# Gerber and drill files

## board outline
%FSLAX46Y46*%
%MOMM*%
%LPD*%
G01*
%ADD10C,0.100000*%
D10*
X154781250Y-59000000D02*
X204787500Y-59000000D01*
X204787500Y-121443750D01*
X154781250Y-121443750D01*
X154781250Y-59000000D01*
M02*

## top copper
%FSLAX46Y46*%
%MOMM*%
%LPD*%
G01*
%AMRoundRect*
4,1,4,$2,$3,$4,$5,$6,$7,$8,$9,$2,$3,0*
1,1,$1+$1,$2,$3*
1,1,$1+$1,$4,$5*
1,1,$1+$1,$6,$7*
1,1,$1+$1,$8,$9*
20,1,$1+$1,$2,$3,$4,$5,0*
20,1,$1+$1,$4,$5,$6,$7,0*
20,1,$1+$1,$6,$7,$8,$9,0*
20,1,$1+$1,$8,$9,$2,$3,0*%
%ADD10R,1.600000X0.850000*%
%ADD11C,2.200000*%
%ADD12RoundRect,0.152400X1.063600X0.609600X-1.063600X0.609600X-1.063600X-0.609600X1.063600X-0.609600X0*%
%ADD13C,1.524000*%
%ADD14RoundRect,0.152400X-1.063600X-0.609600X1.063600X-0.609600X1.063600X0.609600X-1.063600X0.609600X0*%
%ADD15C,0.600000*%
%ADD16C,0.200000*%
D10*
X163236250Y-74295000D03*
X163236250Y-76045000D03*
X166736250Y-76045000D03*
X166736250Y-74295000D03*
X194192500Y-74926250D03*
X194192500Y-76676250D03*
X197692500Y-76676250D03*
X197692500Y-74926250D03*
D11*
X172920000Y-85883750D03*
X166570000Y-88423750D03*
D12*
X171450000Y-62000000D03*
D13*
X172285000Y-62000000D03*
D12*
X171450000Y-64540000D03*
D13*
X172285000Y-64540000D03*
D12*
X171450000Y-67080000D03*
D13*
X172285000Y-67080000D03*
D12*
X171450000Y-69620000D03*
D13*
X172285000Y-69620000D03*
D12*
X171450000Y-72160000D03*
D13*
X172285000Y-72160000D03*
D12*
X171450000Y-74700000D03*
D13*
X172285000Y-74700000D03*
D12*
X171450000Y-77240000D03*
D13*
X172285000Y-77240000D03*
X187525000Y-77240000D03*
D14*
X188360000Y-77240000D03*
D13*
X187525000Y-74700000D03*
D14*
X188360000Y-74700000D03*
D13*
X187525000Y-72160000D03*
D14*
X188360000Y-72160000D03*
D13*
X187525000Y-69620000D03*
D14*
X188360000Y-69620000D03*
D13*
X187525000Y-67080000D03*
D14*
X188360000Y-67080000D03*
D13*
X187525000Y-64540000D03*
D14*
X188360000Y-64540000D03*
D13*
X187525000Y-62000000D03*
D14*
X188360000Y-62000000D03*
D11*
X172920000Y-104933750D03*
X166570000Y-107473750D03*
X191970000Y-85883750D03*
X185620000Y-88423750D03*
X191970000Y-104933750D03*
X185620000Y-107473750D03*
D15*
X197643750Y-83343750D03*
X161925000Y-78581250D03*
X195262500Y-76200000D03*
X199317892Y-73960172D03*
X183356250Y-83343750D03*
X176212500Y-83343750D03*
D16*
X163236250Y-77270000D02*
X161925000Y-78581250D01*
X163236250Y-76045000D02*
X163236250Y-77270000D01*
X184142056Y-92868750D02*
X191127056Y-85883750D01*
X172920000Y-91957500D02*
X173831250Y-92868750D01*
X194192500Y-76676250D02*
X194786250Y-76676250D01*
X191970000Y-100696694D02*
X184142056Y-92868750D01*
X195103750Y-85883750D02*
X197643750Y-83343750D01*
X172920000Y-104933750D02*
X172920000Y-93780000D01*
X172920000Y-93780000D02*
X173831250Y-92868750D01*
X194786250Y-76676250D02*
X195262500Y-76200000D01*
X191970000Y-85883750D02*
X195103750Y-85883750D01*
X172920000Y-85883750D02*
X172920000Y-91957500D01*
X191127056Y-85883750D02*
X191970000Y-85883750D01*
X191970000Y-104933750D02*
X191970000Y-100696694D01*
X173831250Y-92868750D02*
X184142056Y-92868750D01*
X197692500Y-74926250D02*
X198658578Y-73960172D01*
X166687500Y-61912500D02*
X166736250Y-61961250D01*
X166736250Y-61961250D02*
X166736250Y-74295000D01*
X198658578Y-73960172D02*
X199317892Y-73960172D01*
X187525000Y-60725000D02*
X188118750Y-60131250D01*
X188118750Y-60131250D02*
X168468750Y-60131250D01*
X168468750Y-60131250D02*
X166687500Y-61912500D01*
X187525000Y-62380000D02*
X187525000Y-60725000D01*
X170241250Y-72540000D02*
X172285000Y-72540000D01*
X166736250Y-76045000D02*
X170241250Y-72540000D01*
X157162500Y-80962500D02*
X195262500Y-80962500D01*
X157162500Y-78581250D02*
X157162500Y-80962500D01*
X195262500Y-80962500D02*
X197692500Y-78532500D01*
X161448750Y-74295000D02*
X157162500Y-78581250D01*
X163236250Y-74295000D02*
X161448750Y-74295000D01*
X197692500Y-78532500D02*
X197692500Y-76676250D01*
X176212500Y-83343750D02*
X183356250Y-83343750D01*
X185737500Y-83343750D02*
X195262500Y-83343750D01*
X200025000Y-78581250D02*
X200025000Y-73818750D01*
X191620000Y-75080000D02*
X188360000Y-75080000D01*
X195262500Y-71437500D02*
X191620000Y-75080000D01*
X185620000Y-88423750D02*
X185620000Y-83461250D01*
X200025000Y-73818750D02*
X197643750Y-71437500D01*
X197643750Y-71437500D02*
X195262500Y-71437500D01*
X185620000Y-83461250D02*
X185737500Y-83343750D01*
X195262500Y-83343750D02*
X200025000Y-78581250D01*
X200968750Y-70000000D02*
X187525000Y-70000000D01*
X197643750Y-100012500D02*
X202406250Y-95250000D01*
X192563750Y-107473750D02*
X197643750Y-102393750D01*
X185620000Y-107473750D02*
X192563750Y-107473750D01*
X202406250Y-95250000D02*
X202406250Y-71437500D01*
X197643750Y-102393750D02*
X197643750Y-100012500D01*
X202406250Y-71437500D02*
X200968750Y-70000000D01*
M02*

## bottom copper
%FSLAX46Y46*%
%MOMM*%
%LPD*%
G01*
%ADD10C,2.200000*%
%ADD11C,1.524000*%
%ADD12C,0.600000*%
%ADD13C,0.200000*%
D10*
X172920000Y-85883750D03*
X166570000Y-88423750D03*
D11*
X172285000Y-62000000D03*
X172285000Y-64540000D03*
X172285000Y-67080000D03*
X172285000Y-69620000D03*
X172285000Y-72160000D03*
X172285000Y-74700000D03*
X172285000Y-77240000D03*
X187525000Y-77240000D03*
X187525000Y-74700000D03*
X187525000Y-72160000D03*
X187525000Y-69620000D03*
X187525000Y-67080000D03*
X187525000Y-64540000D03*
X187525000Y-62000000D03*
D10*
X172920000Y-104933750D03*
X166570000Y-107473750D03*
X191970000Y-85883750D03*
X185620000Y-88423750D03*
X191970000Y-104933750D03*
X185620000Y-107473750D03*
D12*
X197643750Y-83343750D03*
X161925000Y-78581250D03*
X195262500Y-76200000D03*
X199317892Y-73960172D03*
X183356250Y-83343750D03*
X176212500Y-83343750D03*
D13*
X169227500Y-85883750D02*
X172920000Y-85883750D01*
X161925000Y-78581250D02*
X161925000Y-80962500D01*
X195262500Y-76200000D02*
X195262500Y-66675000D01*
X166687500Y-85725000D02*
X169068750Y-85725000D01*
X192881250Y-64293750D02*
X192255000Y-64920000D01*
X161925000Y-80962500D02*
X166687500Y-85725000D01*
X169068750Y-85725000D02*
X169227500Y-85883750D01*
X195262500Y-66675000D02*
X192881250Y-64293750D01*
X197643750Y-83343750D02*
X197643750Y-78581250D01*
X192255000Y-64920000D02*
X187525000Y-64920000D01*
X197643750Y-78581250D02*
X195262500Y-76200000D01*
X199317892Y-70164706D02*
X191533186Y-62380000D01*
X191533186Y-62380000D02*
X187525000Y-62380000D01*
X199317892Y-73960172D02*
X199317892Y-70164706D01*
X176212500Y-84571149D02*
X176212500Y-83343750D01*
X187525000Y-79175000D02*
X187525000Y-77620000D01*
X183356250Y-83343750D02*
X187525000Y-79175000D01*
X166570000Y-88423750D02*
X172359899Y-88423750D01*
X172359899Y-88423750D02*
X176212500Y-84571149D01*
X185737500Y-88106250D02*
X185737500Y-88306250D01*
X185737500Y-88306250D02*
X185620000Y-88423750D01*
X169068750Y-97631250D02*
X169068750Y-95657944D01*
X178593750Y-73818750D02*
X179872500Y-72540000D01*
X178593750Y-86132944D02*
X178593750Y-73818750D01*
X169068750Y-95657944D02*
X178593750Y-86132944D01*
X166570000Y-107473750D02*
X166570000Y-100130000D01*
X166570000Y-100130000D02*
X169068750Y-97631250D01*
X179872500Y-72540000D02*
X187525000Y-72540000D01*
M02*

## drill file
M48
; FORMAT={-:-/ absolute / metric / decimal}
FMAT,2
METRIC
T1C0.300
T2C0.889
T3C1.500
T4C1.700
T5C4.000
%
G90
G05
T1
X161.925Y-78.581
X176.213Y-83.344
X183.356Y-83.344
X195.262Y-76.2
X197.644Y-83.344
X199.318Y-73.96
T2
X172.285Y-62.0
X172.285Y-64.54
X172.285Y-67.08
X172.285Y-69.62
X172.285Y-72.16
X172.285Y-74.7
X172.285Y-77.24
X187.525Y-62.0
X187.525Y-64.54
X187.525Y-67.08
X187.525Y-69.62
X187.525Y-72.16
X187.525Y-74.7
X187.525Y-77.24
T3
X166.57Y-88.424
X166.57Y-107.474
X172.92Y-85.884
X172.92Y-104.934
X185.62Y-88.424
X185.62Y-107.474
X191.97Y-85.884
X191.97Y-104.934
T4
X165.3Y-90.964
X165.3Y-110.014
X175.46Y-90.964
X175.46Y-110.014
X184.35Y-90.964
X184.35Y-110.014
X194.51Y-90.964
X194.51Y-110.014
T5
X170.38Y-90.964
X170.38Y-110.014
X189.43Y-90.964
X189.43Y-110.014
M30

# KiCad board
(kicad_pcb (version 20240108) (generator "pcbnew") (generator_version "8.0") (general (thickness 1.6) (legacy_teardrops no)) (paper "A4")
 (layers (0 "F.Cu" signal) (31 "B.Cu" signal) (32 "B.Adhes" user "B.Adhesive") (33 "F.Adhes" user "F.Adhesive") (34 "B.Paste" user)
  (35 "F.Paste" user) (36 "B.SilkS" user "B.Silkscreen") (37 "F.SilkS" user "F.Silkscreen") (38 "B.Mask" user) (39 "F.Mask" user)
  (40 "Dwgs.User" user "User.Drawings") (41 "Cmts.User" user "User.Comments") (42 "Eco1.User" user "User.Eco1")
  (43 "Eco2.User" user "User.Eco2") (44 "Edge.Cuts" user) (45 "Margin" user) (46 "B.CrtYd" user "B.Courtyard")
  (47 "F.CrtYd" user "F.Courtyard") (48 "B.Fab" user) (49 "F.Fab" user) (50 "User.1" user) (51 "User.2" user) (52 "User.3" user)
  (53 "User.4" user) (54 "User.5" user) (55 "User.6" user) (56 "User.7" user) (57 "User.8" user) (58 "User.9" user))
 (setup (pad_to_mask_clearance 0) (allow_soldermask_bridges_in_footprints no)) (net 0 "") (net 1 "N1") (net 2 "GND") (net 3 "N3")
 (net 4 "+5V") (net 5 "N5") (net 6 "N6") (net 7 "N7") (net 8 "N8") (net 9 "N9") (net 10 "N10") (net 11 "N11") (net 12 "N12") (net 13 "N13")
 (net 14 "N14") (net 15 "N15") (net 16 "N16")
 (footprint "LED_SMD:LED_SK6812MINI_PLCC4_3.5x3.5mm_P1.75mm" (layer "F.Cu") (at 164.98625 75.17)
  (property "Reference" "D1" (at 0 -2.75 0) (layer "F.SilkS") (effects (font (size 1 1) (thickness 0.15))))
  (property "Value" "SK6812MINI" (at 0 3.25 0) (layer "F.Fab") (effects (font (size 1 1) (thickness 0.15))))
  (pad "1" smd rect (at -1.75 -0.875) (size 1.6 0.85) (layers "F.Cu" "F.Paste" "F.Mask") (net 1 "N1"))
  (pad "2" smd rect (at -1.75 0.875) (size 1.6 0.85) (layers "F.Cu" "F.Paste" "F.Mask") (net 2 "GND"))
  (pad "3" smd rect (at 1.75 0.875) (size 1.6 0.85) (layers "F.Cu" "F.Paste" "F.Mask") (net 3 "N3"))
  (pad "4" smd rect (at 1.75 -0.875) (size 1.6 0.85) (layers "F.Cu" "F.Paste" "F.Mask") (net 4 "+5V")))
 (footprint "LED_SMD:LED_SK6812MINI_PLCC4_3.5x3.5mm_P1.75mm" (layer "F.Cu") (at 195.9425 75.80125)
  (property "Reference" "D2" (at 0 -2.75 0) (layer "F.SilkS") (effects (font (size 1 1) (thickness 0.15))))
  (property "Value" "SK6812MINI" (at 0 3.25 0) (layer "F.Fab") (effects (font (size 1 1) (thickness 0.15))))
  (pad "1" smd rect (at -1.75 -0.875) (size 1.6 0.85) (layers "F.Cu" "F.Paste" "F.Mask") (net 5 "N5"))
  (pad "2" smd rect (at -1.75 0.875) (size 1.6 0.85) (layers "F.Cu" "F.Paste" "F.Mask") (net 2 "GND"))
  (pad "3" smd rect (at 1.75 0.875) (size 1.6 0.85) (layers "F.Cu" "F.Paste" "F.Mask") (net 1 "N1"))
  (pad "4" smd rect (at 1.75 -0.875) (size 1.6 0.85) (layers "F.Cu" "F.Paste" "F.Mask") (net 4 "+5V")))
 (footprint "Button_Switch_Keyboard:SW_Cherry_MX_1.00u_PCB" (layer "F.Cu") (at 172.92 85.88375)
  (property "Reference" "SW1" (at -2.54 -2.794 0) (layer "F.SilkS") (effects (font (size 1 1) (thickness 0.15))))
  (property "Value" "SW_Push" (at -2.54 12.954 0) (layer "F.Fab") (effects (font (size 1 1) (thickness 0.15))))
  (pad "" np_thru_hole circle (at -7.62 5.08) (size 1.7 1.7) (drill 1.7) (layers "*.Cu" "*.Mask"))
  (pad "" np_thru_hole circle (at -2.54 5.08) (size 4 4) (drill 4) (layers "*.Cu" "*.Mask"))
  (pad "" np_thru_hole circle (at 2.54 5.08) (size 1.7 1.7) (drill 1.7) (layers "*.Cu" "*.Mask"))
  (pad "1" thru_hole circle (at 0 0) (size 2.2 2.2) (drill 1.5) (layers "*.Cu" "*.Mask") (remove_unused_layers no) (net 2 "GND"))
  (pad "2" thru_hole circle (at -6.35 2.54) (size 2.2 2.2) (drill 1.5) (layers "*.Cu" "*.Mask") (remove_unused_layers no) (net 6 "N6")))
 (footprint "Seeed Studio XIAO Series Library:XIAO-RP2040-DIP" (layer "F.Cu") (at 179.905 69.62)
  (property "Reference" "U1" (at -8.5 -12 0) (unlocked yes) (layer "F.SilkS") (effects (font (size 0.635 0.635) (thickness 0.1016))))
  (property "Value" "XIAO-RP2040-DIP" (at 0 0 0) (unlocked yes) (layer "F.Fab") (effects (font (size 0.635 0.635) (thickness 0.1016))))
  (pad "1" smd roundrect (at -8.455 -7.62 180) (size 2.432 1.524) (layers "F.Cu" "F.Mask") (roundrect_rratio 0.1) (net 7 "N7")
   (thermal_bridge_angle 45))
  (pad "1" thru_hole circle (at -7.62 -7.62 180) (size 1.524 1.524) (drill 0.889) (layers "*.Cu" "*.Mask") (remove_unused_layers no)
   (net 7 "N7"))
  (pad "2" smd roundrect (at -8.455 -5.08 180) (size 2.432 1.524) (layers "F.Cu" "F.Mask") (roundrect_rratio 0.1) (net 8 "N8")
   (thermal_bridge_angle 45))
  (pad "2" thru_hole circle (at -7.62 -5.08 180) (size 1.524 1.524) (drill 0.889) (layers "*.Cu" "*.Mask") (remove_unused_layers no)
   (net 8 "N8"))
  (pad "3" smd roundrect (at -8.455 -2.54 180) (size 2.432 1.524) (layers "F.Cu" "F.Mask") (roundrect_rratio 0.1) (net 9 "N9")
   (thermal_bridge_angle 45))
  (pad "3" thru_hole circle (at -7.62 -2.54 180) (size 1.524 1.524) (drill 0.889) (layers "*.Cu" "*.Mask") (remove_unused_layers no)
   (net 9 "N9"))
  (pad "4" smd roundrect (at -8.455 0 180) (size 2.432 1.524) (layers "F.Cu" "F.Mask") (roundrect_rratio 0.1) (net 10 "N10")
   (thermal_bridge_angle 45))
  (pad "4" thru_hole circle (at -7.62 0 180) (size 1.524 1.524) (drill 0.889) (layers "*.Cu" "*.Mask") (remove_unused_layers no)
   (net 10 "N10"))
  (pad "5" smd roundrect (at -8.455 2.54 180) (size 2.432 1.524) (layers "F.Cu" "F.Mask") (roundrect_rratio 0.1) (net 3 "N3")
   (thermal_bridge_angle 45))
  (pad "5" thru_hole circle (at -7.62 2.54 180) (size 1.524 1.524) (drill 0.889) (layers "*.Cu" "*.Mask") (remove_unused_layers no)
   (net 3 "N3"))
  (pad "6" smd roundrect (at -8.455 5.08 180) (size 2.432 1.524) (layers "F.Cu" "F.Mask") (roundrect_rratio 0.1) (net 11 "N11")
   (thermal_bridge_angle 45))
  (pad "6" thru_hole circle (at -7.62 5.08 180) (size 1.524 1.524) (drill 0.889) (layers "*.Cu" "*.Mask") (remove_unused_layers no)
   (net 11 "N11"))
  (pad "7" smd roundrect (at -8.455 7.62 180) (size 2.432 1.524) (layers "F.Cu" "F.Mask") (roundrect_rratio 0.1) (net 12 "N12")
   (thermal_bridge_angle 45))
  (pad "7" thru_hole circle (at -7.62 7.62 180) (size 1.524 1.524) (drill 0.889) (layers "*.Cu" "*.Mask") (remove_unused_layers no)
   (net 12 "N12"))
  (pad "8" thru_hole circle (at 7.62 7.62) (size 1.524 1.524) (drill 0.889) (layers "*.Cu" "*.Mask") (remove_unused_layers no) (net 6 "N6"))
  (pad "8" smd roundrect (at 8.455 7.62) (size 2.432 1.524) (layers "F.Cu" "F.Mask") (roundrect_rratio 0.1) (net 6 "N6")
   (thermal_bridge_angle 45))
  (pad "9" thru_hole circle (at 7.62 5.08) (size 1.524 1.524) (drill 0.889) (layers "*.Cu" "*.Mask") (remove_unused_layers no)
   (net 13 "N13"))
  (pad "9" smd roundrect (at 8.455 5.08) (size 2.432 1.524) (layers "F.Cu" "F.Mask") (roundrect_rratio 0.1) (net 13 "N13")
   (thermal_bridge_angle 45))
  (pad "10" thru_hole circle (at 7.62 2.54) (size 1.524 1.524) (drill 0.889) (layers "*.Cu" "*.Mask") (remove_unused_layers no)
   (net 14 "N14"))
  (pad "10" smd roundrect (at 8.455 2.54) (size 2.432 1.524) (layers "F.Cu" "F.Mask") (roundrect_rratio 0.1) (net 14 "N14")
   (thermal_bridge_angle 45))
  (pad "11" thru_hole circle (at 7.62 0) (size 1.524 1.524) (drill 0.889) (layers "*.Cu" "*.Mask") (remove_unused_layers no) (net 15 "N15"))
  (pad "11" smd roundrect (at 8.455 0) (size 2.432 1.524) (layers "F.Cu" "F.Mask") (roundrect_rratio 0.1) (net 15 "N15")
   (thermal_bridge_angle 45))
  (pad "12" thru_hole circle (at 7.62 -2.54) (size 1.524 1.524) (drill 0.889) (layers "*.Cu" "*.Mask") (remove_unused_layers no)
   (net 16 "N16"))
  (pad "12" smd roundrect (at 8.455 -2.54) (size 2.432 1.524) (layers "F.Cu" "F.Mask") (roundrect_rratio 0.1) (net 16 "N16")
   (thermal_bridge_angle 45))
  (pad "13" thru_hole circle (at 7.62 -5.08) (size 1.524 1.524) (drill 0.889) (layers "*.Cu" "*.Mask") (remove_unused_layers no)
   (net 2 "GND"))
  (pad "13" smd roundrect (at 8.455 -5.08) (size 2.432 1.524) (layers "F.Cu" "F.Mask") (roundrect_rratio 0.1) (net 2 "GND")
   (thermal_bridge_angle 45))
  (pad "14" thru_hole circle (at 7.62 -7.62) (size 1.524 1.524) (drill 0.889) (layers "*.Cu" "*.Mask") (remove_unused_layers no)
   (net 4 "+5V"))
  (pad "14" smd roundrect (at 8.455 -7.62) (size 2.432 1.524) (layers "F.Cu" "F.Mask") (roundrect_rratio 0.1) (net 4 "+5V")
   (thermal_bridge_angle 45)))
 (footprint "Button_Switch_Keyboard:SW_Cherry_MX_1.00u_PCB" (layer "F.Cu") (at 172.92 104.93375)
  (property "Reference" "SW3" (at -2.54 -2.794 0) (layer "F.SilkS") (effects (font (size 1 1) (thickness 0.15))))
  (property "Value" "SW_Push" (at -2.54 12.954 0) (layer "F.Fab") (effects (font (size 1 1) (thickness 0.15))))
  (pad "" np_thru_hole circle (at -7.62 5.08) (size 1.7 1.7) (drill 1.7) (layers "*.Cu" "*.Mask"))
  (pad "" np_thru_hole circle (at -2.54 5.08) (size 4 4) (drill 4) (layers "*.Cu" "*.Mask"))
  (pad "" np_thru_hole circle (at 2.54 5.08) (size 1.7 1.7) (drill 1.7) (layers "*.Cu" "*.Mask"))
  (pad "1" thru_hole circle (at 0 0) (size 2.2 2.2) (drill 1.5) (layers "*.Cu" "*.Mask") (remove_unused_layers no) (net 2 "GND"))
  (pad "2" thru_hole circle (at -6.35 2.54) (size 2.2 2.2) (drill 1.5) (layers "*.Cu" "*.Mask") (remove_unused_layers no) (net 14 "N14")))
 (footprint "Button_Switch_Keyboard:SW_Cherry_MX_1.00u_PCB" (layer "F.Cu") (at 191.97 85.88375)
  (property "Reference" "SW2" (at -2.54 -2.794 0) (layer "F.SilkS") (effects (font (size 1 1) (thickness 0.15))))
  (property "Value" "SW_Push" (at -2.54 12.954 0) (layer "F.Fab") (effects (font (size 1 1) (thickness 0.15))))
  (pad "" np_thru_hole circle (at -7.62 5.08) (size 1.7 1.7) (drill 1.7) (layers "*.Cu" "*.Mask"))
  (pad "" np_thru_hole circle (at -2.54 5.08) (size 4 4) (drill 4) (layers "*.Cu" "*.Mask"))
  (pad "" np_thru_hole circle (at 2.54 5.08) (size 1.7 1.7) (drill 1.7) (layers "*.Cu" "*.Mask"))
  (pad "1" thru_hole circle (at 0 0) (size 2.2 2.2) (drill 1.5) (layers "*.Cu" "*.Mask") (remove_unused_layers no) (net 2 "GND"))
  (pad "2" thru_hole circle (at -6.35 2.54) (size 2.2 2.2) (drill 1.5) (layers "*.Cu" "*.Mask") (remove_unused_layers no) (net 13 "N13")))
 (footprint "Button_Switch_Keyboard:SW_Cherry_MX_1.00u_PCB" (layer "F.Cu") (at 191.97 104.93375)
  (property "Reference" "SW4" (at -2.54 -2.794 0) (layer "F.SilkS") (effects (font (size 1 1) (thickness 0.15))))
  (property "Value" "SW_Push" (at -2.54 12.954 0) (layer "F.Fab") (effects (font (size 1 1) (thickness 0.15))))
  (pad "" np_thru_hole circle (at -7.62 5.08) (size 1.7 1.7) (drill 1.7) (layers "*.Cu" "*.Mask"))
  (pad "" np_thru_hole circle (at -2.54 5.08) (size 4 4) (drill 4) (layers "*.Cu" "*.Mask"))
  (pad "" np_thru_hole circle (at 2.54 5.08) (size 1.7 1.7) (drill 1.7) (layers "*.Cu" "*.Mask"))
  (pad "1" thru_hole circle (at 0 0) (size 2.2 2.2) (drill 1.5) (layers "*.Cu" "*.Mask") (remove_unused_layers no) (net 2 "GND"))
  (pad "2" thru_hole circle (at -6.35 2.54) (size 2.2 2.2) (drill 1.5) (layers "*.Cu" "*.Mask") (remove_unused_layers no) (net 15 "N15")))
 (gr_rect (start 154.78125 59) (end 204.7875 121.44375) (stroke (width 0.1) (type default)) (fill none) (layer "Edge.Cuts"))
 (segment (start 163.23625 77.27) (end 161.925 78.58125) (width 0.2) (layer "F.Cu") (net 2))
 (segment (start 163.23625 76.045) (end 163.23625 77.27) (width 0.2) (layer "F.Cu") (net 2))
 (segment (start 184.142056 92.86875) (end 191.127056 85.88375) (width 0.2) (layer "F.Cu") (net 2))
 (segment (start 172.92 91.9575) (end 173.83125 92.86875) (width 0.2) (layer "F.Cu") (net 2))
 (segment (start 194.1925 76.67625) (end 194.78625 76.67625) (width 0.2) (layer "F.Cu") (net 2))
 (segment (start 191.97 100.696694) (end 184.142056 92.86875) (width 0.2) (layer "F.Cu") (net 2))
 (segment (start 195.10375 85.88375) (end 197.64375 83.34375) (width 0.2) (layer "F.Cu") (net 2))
 (segment (start 172.92 104.93375) (end 172.92 93.78) (width 0.2) (layer "F.Cu") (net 2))
 (segment (start 172.92 93.78) (end 173.83125 92.86875) (width 0.2) (layer "F.Cu") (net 2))
 (segment (start 194.78625 76.67625) (end 195.2625 76.2) (width 0.2) (layer "F.Cu") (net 2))
 (segment (start 191.97 85.88375) (end 195.10375 85.88375) (width 0.2) (layer "F.Cu") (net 2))
 (segment (start 172.92 85.88375) (end 172.92 91.9575) (width 0.2) (layer "F.Cu") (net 2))
 (segment (start 191.127056 85.88375) (end 191.97 85.88375) (width 0.2) (layer "F.Cu") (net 2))
 (segment (start 191.97 104.93375) (end 191.97 100.696694) (width 0.2) (layer "F.Cu") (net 2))
 (segment (start 173.83125 92.86875) (end 184.142056 92.86875) (width 0.2) (layer "F.Cu") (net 2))
 (via (at 197.64375 83.34375) (size 0.6) (drill 0.3) (layers "F.Cu" "B.Cu") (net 2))
 (via (at 161.925 78.58125) (size 0.6) (drill 0.3) (layers "F.Cu" "B.Cu") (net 2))
 (via (at 195.2625 76.2) (size 0.6) (drill 0.3) (layers "F.Cu" "B.Cu") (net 2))
 (segment (start 169.2275 85.88375) (end 172.92 85.88375) (width 0.2) (layer "B.Cu") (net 2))
 (segment (start 161.925 78.58125) (end 161.925 80.9625) (width 0.2) (layer "B.Cu") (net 2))
 (segment (start 195.2625 76.2) (end 195.2625 66.675) (width 0.2) (layer "B.Cu") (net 2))
 (segment (start 166.6875 85.725) (end 169.06875 85.725) (width 0.2) (layer "B.Cu") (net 2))
 (segment (start 192.88125 64.29375) (end 192.255 64.92) (width 0.2) (layer "B.Cu") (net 2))
 (segment (start 161.925 80.9625) (end 166.6875 85.725) (width 0.2) (layer "B.Cu") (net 2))
 (segment (start 169.06875 85.725) (end 169.2275 85.88375) (width 0.2) (layer "B.Cu") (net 2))
 (segment (start 195.2625 66.675) (end 192.88125 64.29375) (width 0.2) (layer "B.Cu") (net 2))
 (segment (start 197.64375 83.34375) (end 197.64375 78.58125) (width 0.2) (layer "B.Cu") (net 2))
 (segment (start 192.255 64.92) (end 187.525 64.92) (width 0.2) (layer "B.Cu") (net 2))
 (segment (start 197.64375 78.58125) (end 195.2625 76.2) (width 0.2) (layer "B.Cu") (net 2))
 (segment (start 197.6925 74.92625) (end 198.658578 73.960172) (width 0.2) (layer "F.Cu") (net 4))
 (segment (start 166.6875 61.9125) (end 166.73625 61.96125) (width 0.2) (layer "F.Cu") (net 4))
 (segment (start 166.73625 61.96125) (end 166.73625 74.295) (width 0.2) (layer "F.Cu") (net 4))
 (segment (start 198.658578 73.960172) (end 199.317892 73.960172) (width 0.2) (layer "F.Cu") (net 4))
 (segment (start 187.525 60.725) (end 188.11875 60.13125) (width 0.2) (layer "F.Cu") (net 4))
 (segment (start 188.11875 60.13125) (end 168.46875 60.13125) (width 0.2) (layer "F.Cu") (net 4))
 (segment (start 168.46875 60.13125) (end 166.6875 61.9125) (width 0.2) (layer "F.Cu") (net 4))
 (segment (start 187.525 62.38) (end 187.525 60.725) (width 0.2) (layer "F.Cu") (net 4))
 (via (at 199.317892 73.960172) (size 0.6) (drill 0.3) (layers "F.Cu" "B.Cu") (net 4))
 (segment (start 199.317892 70.164706) (end 191.533186 62.38) (width 0.2) (layer "B.Cu") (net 4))
 (segment (start 191.533186 62.38) (end 187.525 62.38) (width 0.2) (layer "B.Cu") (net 4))
 (segment (start 199.317892 73.960172) (end 199.317892 70.164706) (width 0.2) (layer "B.Cu") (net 4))
 (segment (start 170.24125 72.54) (end 172.285 72.54) (width 0.2) (layer "F.Cu") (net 3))
 (segment (start 166.73625 76.045) (end 170.24125 72.54) (width 0.2) (layer "F.Cu") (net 3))
 (segment (start 157.1625 80.9625) (end 195.2625 80.9625) (width 0.2) (layer "F.Cu") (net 1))
 (segment (start 157.1625 78.58125) (end 157.1625 80.9625) (width 0.2) (layer "F.Cu") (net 1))
 (segment (start 195.2625 80.9625) (end 197.6925 78.5325) (width 0.2) (layer "F.Cu") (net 1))
 (segment (start 161.44875 74.295) (end 157.1625 78.58125) (width 0.2) (layer "F.Cu") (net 1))
 (segment (start 163.23625 74.295) (end 161.44875 74.295) (width 0.2) (layer "F.Cu") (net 1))
 (segment (start 197.6925 78.5325) (end 197.6925 76.67625) (width 0.2) (layer "F.Cu") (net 1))
 (segment (start 176.2125 83.34375) (end 183.35625 83.34375) (width 0.2) (layer "F.Cu") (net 6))
 (via (at 183.35625 83.34375) (size 0.6) (drill 0.3) (layers "F.Cu" "B.Cu") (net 6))
 (via (at 176.2125 83.34375) (size 0.6) (drill 0.3) (layers "F.Cu" "B.Cu") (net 6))
 (segment (start 176.2125 84.571149) (end 176.2125 83.34375) (width 0.2) (layer "B.Cu") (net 6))
 (segment (start 187.525 79.175) (end 187.525 77.62) (width 0.2) (layer "B.Cu") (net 6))
 (segment (start 183.35625 83.34375) (end 187.525 79.175) (width 0.2) (layer "B.Cu") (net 6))
 (segment (start 166.57 88.42375) (end 172.359899 88.42375) (width 0.2) (layer "B.Cu") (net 6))
 (segment (start 172.359899 88.42375) (end 176.2125 84.571149) (width 0.2) (layer "B.Cu") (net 6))
 (segment (start 185.7375 83.34375) (end 195.2625 83.34375) (width 0.2) (layer "F.Cu") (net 13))
 (segment (start 200.025 78.58125) (end 200.025 73.81875) (width 0.2) (layer "F.Cu") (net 13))
 (segment (start 191.62 75.08) (end 188.36 75.08) (width 0.2) (layer "F.Cu") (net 13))
 (segment (start 195.2625 71.4375) (end 191.62 75.08) (width 0.2) (layer "F.Cu") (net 13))
 (segment (start 185.62 88.42375) (end 185.62 83.46125) (width 0.2) (layer "F.Cu") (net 13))
 (segment (start 200.025 73.81875) (end 197.64375 71.4375) (width 0.2) (layer "F.Cu") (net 13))
 (segment (start 197.64375 71.4375) (end 195.2625 71.4375) (width 0.2) (layer "F.Cu") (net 13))
 (segment (start 185.62 83.46125) (end 185.7375 83.34375) (width 0.2) (layer "F.Cu") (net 13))
 (segment (start 195.2625 83.34375) (end 200.025 78.58125) (width 0.2) (layer "F.Cu") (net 13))
 (segment (start 185.7375 88.10625) (end 185.7375 88.30625) (width 0.2) (layer "B.Cu") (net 13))
 (segment (start 185.7375 88.30625) (end 185.62 88.42375) (width 0.2) (layer "B.Cu") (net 13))
 (segment (start 169.06875 97.63125) (end 169.06875 95.657944) (width 0.2) (layer "B.Cu") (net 14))
 (segment (start 178.59375 73.81875) (end 179.8725 72.54) (width 0.2) (layer "B.Cu") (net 14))
 (segment (start 178.59375 86.132944) (end 178.59375 73.81875) (width 0.2) (layer "B.Cu") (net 14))
 (segment (start 169.06875 95.657944) (end 178.59375 86.132944) (width 0.2) (layer "B.Cu") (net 14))
 (segment (start 166.57 107.47375) (end 166.57 100.13) (width 0.2) (layer "B.Cu") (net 14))
 (segment (start 166.57 100.13) (end 169.06875 97.63125) (width 0.2) (layer "B.Cu") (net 14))
 (segment (start 179.8725 72.54) (end 187.525 72.54) (width 0.2) (layer "B.Cu") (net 14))
 (segment (start 200.96875 70) (end 187.525 70) (width 0.2) (layer "F.Cu") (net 15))
 (segment (start 197.64375 100.0125) (end 202.40625 95.25) (width 0.2) (layer "F.Cu") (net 15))
 (segment (start 192.56375 107.47375) (end 197.64375 102.39375) (width 0.2) (layer "F.Cu") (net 15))
 (segment (start 185.62 107.47375) (end 192.56375 107.47375) (width 0.2) (layer "F.Cu") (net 15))
 (segment (start 202.40625 95.25) (end 202.40625 71.4375) (width 0.2) (layer "F.Cu") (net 15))
 (segment (start 197.64375 102.39375) (end 197.64375 100.0125) (width 0.2) (layer "F.Cu") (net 15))
 (segment (start 202.40625 71.4375) (end 200.96875 70) (width 0.2) (layer "F.Cu") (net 15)))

